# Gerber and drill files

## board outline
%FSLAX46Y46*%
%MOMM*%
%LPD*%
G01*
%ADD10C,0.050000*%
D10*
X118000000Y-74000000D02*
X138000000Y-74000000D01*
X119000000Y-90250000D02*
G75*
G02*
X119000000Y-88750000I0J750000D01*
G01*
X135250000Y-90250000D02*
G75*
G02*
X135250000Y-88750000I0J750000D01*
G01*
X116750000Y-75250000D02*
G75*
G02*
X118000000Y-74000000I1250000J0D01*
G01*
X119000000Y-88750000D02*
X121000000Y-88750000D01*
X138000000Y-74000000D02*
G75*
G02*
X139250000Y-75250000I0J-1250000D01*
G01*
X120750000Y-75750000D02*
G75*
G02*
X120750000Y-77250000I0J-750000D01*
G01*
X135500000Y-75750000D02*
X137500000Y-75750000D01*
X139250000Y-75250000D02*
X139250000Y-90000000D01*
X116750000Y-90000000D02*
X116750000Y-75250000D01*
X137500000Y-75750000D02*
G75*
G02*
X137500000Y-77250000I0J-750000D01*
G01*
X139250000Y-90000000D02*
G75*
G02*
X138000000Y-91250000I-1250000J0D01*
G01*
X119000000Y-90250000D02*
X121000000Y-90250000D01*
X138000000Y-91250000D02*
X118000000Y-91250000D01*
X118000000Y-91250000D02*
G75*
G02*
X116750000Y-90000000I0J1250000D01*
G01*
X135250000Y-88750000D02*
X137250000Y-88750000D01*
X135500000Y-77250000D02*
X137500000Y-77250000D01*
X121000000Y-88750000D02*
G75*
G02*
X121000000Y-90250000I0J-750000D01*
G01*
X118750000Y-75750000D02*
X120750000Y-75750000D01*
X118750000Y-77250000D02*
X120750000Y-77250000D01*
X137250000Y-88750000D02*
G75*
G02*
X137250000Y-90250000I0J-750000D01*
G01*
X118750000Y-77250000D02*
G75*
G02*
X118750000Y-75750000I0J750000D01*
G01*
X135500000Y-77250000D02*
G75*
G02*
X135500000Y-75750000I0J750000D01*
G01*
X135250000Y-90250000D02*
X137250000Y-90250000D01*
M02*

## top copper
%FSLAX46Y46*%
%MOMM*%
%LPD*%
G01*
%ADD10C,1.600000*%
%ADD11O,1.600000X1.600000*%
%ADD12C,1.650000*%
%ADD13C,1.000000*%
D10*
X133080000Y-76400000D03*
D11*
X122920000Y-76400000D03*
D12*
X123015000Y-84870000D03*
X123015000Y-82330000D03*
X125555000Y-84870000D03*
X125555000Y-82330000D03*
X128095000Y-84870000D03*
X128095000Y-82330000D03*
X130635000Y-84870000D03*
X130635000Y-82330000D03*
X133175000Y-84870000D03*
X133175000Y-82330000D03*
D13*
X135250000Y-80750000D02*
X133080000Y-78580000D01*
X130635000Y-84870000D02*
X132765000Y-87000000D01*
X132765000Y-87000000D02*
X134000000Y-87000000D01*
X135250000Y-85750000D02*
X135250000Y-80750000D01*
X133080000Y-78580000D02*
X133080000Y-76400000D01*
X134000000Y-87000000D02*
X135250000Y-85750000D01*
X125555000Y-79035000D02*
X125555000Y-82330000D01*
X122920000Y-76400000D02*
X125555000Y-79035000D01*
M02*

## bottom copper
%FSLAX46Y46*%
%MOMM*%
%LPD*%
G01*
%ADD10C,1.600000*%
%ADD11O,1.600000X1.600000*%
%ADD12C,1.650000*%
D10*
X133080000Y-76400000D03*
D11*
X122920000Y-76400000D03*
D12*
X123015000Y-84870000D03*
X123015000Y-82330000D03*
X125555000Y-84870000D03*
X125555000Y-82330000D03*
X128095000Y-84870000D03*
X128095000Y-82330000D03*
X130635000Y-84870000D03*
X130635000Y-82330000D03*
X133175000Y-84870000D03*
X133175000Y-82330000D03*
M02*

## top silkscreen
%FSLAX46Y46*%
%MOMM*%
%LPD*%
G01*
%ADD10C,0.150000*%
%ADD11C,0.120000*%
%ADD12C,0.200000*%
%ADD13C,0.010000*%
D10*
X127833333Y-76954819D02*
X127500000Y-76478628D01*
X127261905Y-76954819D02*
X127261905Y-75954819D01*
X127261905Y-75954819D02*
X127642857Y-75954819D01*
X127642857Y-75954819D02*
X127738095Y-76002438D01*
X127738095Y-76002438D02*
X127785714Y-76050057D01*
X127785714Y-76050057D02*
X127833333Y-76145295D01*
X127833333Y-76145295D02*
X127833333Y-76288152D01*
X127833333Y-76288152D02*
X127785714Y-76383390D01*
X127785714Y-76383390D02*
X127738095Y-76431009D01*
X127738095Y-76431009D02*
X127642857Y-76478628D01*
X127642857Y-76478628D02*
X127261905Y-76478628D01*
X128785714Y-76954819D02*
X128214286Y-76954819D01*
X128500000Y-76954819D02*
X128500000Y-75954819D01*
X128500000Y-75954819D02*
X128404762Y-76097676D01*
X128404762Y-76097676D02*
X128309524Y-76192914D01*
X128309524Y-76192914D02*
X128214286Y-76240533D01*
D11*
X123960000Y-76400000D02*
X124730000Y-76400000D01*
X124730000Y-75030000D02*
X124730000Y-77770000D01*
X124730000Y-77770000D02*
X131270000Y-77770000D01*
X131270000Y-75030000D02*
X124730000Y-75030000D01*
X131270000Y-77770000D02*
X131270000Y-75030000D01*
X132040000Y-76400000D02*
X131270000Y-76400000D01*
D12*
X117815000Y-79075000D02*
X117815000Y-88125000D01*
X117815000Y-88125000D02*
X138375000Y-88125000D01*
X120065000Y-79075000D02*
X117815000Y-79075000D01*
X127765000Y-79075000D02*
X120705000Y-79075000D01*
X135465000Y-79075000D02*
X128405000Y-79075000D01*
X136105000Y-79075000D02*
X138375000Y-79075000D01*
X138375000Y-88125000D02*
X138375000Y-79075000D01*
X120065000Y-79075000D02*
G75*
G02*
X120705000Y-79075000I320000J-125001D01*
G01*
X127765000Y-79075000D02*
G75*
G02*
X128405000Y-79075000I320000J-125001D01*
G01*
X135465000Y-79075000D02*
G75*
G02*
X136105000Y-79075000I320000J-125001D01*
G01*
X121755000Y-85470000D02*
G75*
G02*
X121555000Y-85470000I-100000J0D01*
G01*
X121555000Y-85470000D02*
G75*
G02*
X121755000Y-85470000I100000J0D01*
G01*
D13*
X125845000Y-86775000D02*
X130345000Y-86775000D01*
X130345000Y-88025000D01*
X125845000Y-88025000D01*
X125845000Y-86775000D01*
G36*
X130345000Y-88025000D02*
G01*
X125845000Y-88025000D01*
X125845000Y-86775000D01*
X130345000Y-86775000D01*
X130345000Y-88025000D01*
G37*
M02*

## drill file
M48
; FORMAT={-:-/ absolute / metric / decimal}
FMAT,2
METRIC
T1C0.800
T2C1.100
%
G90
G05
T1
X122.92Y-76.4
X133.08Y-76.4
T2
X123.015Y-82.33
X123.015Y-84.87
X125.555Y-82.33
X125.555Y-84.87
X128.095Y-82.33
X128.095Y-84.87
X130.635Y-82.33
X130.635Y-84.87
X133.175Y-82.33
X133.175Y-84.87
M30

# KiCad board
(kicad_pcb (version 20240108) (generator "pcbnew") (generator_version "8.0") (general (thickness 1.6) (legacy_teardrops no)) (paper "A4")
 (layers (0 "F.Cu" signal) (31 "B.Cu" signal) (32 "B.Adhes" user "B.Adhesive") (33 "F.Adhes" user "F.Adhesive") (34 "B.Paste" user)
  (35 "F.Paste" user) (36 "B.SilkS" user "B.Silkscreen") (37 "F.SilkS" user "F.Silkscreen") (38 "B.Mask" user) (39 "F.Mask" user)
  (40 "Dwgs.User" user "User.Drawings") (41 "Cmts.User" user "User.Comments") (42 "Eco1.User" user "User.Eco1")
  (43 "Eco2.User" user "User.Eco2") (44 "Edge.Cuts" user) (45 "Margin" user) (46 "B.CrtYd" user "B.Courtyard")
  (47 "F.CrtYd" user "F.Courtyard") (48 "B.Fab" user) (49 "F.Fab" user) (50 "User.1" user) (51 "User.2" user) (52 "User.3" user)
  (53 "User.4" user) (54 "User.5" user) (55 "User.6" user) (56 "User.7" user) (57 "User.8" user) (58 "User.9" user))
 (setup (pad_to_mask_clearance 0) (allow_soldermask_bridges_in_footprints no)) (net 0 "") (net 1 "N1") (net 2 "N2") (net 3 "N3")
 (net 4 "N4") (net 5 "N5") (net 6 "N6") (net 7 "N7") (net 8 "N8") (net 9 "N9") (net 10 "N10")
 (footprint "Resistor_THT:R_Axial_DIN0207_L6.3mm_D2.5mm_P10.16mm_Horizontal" (layer "F.Cu") (at 133.08 76.4 180)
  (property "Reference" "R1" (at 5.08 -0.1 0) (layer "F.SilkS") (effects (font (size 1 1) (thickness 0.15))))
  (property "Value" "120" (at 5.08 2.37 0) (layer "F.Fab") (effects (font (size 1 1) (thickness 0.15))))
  (fp_line (start 9.12 0) (end 8.35 0) (stroke (width 0.12) (type solid)) (layer "F.SilkS"))
  (fp_line (start 8.35 1.37) (end 8.35 -1.37) (stroke (width 0.12) (type solid)) (layer "F.SilkS"))
  (fp_line (start 8.35 -1.37) (end 1.81 -1.37) (stroke (width 0.12) (type solid)) (layer "F.SilkS"))
  (fp_line (start 1.81 1.37) (end 8.35 1.37) (stroke (width 0.12) (type solid)) (layer "F.SilkS"))
  (fp_line (start 1.81 -1.37) (end 1.81 1.37) (stroke (width 0.12) (type solid)) (layer "F.SilkS"))
  (fp_line (start 1.04 0) (end 1.81 0) (stroke (width 0.12) (type solid)) (layer "F.SilkS"))
  (pad "1" thru_hole circle (at 0 0 180) (size 1.6 1.6) (drill 0.8) (layers "*.Cu" "*.Mask") (remove_unused_layers no) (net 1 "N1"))
  (pad "2" thru_hole oval (at 10.16 0 180) (size 1.6 1.6) (drill 0.8) (layers "*.Cu" "*.Mask") (remove_unused_layers no) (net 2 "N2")))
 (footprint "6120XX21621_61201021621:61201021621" (layer "F.Cu") (at 128.095 83.6)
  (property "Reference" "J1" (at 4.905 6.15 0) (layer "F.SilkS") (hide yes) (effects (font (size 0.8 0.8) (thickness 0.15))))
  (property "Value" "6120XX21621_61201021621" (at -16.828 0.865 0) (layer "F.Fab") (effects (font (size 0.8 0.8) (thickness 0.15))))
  (fp_line (start -10.28 -4.525) (end -10.28 4.525) (stroke (width 0.2) (type solid)) (layer "F.SilkS"))
  (fp_line (start -10.28 4.525) (end 10.28 4.525) (stroke (width 0.2) (type solid)) (layer "F.SilkS"))
  (fp_line (start -8.03 -4.525) (end -10.28 -4.525) (stroke (width 0.2) (type solid)) (layer "F.SilkS"))
  (fp_line (start -0.33 -4.525) (end -7.39 -4.525) (stroke (width 0.2) (type solid)) (layer "F.SilkS"))
  (fp_line (start 7.37 -4.525) (end 0.31 -4.525) (stroke (width 0.2) (type solid)) (layer "F.SilkS"))
  (fp_line (start 8.01 -4.525) (end 10.28 -4.525) (stroke (width 0.2) (type solid)) (layer "F.SilkS"))
  (fp_line (start 10.28 4.525) (end 10.28 -4.525) (stroke (width 0.2) (type solid)) (layer "F.SilkS"))
  (fp_arc (start -8.03 -4.525) (mid -7.71 -4.743547) (end -7.39 -4.525) (stroke (width 0.2) (type solid)) (layer "F.SilkS"))
  (fp_arc (start -0.33 -4.525) (mid -0.01 -4.743547) (end 0.31 -4.525) (stroke (width 0.2) (type solid)) (layer "F.SilkS"))
  (fp_arc (start 7.37 -4.525) (mid 7.69 -4.743547) (end 8.01 -4.525) (stroke (width 0.2) (type solid)) (layer "F.SilkS"))
  (fp_circle (center -6.44 1.87) (end -6.34 1.87) (stroke (width 0.2) (type solid)) (fill none) (layer "F.SilkS"))
  (fp_poly
   (pts (xy -2.25 3.175) (xy 2.25 3.175) (xy 2.25 4.425) (xy -2.25 4.425)) (stroke (width 0.01) (type solid)) (fill solid) (layer "F.SilkS"))
  (pad "1" thru_hole circle (at -5.08 1.27) (size 1.65 1.65) (drill 1.1) (layers "*.Cu" "*.Mask") (remove_unused_layers no) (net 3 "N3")
   (solder_mask_margin 0.102))
  (pad "2" thru_hole circle (at -5.08 -1.27) (size 1.65 1.65) (drill 1.1) (layers "*.Cu" "*.Mask") (remove_unused_layers no) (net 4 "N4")
   (solder_mask_margin 0.102))
  (pad "3" thru_hole circle (at -2.54 1.27) (size 1.65 1.65) (drill 1.1) (layers "*.Cu" "*.Mask") (remove_unused_layers no) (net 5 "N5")
   (solder_mask_margin 0.102))
  (pad "4" thru_hole circle (at -2.54 -1.27) (size 1.65 1.65) (drill 1.1) (layers "*.Cu" "*.Mask") (remove_unused_layers no) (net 2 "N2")
   (solder_mask_margin 0.102))
  (pad "5" thru_hole circle (at 0 1.27) (size 1.65 1.65) (drill 1.1) (layers "*.Cu" "*.Mask") (remove_unused_layers no) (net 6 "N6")
   (solder_mask_margin 0.102))
  (pad "6" thru_hole circle (at 0 -1.27) (size 1.65 1.65) (drill 1.1) (layers "*.Cu" "*.Mask") (remove_unused_layers no) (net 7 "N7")
   (solder_mask_margin 0.102))
  (pad "7" thru_hole circle (at 2.54 1.27) (size 1.65 1.65) (drill 1.1) (layers "*.Cu" "*.Mask") (remove_unused_layers no) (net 1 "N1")
   (solder_mask_margin 0.102))
  (pad "8" thru_hole circle (at 2.54 -1.27) (size 1.65 1.65) (drill 1.1) (layers "*.Cu" "*.Mask") (remove_unused_layers no) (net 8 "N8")
   (solder_mask_margin 0.102))
  (pad "9" thru_hole circle (at 5.08 1.27) (size 1.65 1.65) (drill 1.1) (layers "*.Cu" "*.Mask") (remove_unused_layers no) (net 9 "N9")
   (solder_mask_margin 0.102))
  (pad "10" thru_hole circle (at 5.08 -1.27) (size 1.65 1.65) (drill 1.1) (layers "*.Cu" "*.Mask") (remove_unused_layers no) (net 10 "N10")
   (solder_mask_margin 0.102)))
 (gr_line (start 118 74) (end 138 74) (stroke (width 0.05) (type default)) (layer "Edge.Cuts"))
 (gr_arc (start 119 90.25) (mid 118.25 89.5) (end 119 88.75) (stroke (width 0.05) (type default)) (layer "Edge.Cuts"))
 (gr_arc (start 135.25 90.25) (mid 134.5 89.5) (end 135.25 88.75) (stroke (width 0.05) (type default)) (layer "Edge.Cuts"))
 (gr_arc (start 116.75 75.25) (mid 117.116117 74.366117) (end 118 74) (stroke (width 0.05) (type default)) (layer "Edge.Cuts"))
 (gr_line (start 119 88.75) (end 121 88.75) (stroke (width 0.05) (type default)) (layer "Edge.Cuts"))
 (gr_arc (start 138 74) (mid 138.883883 74.366117) (end 139.25 75.25) (stroke (width 0.05) (type default)) (layer "Edge.Cuts"))
 (gr_arc (start 120.75 75.75) (mid 121.5 76.5) (end 120.75 77.25) (stroke (width 0.05) (type default)) (layer "Edge.Cuts"))
 (gr_line (start 135.5 75.75) (end 137.5 75.75) (stroke (width 0.05) (type default)) (layer "Edge.Cuts"))
 (gr_line (start 139.25 75.25) (end 139.25 90) (stroke (width 0.05) (type default)) (layer "Edge.Cuts"))
 (gr_line (start 116.75 90) (end 116.75 75.25) (stroke (width 0.05) (type default)) (layer "Edge.Cuts"))
 (gr_arc (start 137.5 75.75) (mid 138.25 76.5) (end 137.5 77.25) (stroke (width 0.05) (type default)) (layer "Edge.Cuts"))
 (gr_arc (start 139.25 90) (mid 138.883883 90.883883) (end 138 91.25) (stroke (width 0.05) (type default)) (layer "Edge.Cuts"))
 (gr_line (start 119 90.25) (end 121 90.25) (stroke (width 0.05) (type default)) (layer "Edge.Cuts"))
 (gr_line (start 138 91.25) (end 118 91.25) (stroke (width 0.05) (type default)) (layer "Edge.Cuts"))
 (gr_arc (start 118 91.25) (mid 117.116117 90.883883) (end 116.75 90) (stroke (width 0.05) (type default)) (layer "Edge.Cuts"))
 (gr_line (start 135.25 88.75) (end 137.25 88.75) (stroke (width 0.05) (type default)) (layer "Edge.Cuts"))
 (gr_line (start 135.5 77.25) (end 137.5 77.25) (stroke (width 0.05) (type default)) (layer "Edge.Cuts"))
 (gr_arc (start 121 88.75) (mid 121.75 89.5) (end 121 90.25) (stroke (width 0.05) (type default)) (layer "Edge.Cuts"))
 (gr_line (start 118.75 75.75) (end 120.75 75.75) (stroke (width 0.05) (type default)) (layer "Edge.Cuts"))
 (gr_line (start 118.75 77.25) (end 120.75 77.25) (stroke (width 0.05) (type default)) (layer "Edge.Cuts"))
 (gr_arc (start 137.25 88.75) (mid 138 89.5) (end 137.25 90.25) (stroke (width 0.05) (type default)) (layer "Edge.Cuts"))
 (gr_arc (start 118.75 77.25) (mid 118 76.5) (end 118.75 75.75) (stroke (width 0.05) (type default)) (layer "Edge.Cuts"))
 (gr_arc (start 135.5 77.25) (mid 134.75 76.5) (end 135.5 75.75) (stroke (width 0.05) (type default)) (layer "Edge.Cuts"))
 (gr_line (start 135.25 90.25) (end 137.25 90.25) (stroke (width 0.05) (type default)) (layer "Edge.Cuts"))
 (segment (start 135.25 80.75) (end 133.08 78.58) (width 1) (layer "F.Cu") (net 1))
 (segment (start 130.635 84.87) (end 132.765 87) (width 1) (layer "F.Cu") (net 1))
 (segment (start 132.765 87) (end 134 87) (width 1) (layer "F.Cu") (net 1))
 (segment (start 135.25 85.75) (end 135.25 80.75) (width 1) (layer "F.Cu") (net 1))
 (segment (start 133.08 78.58) (end 133.08 76.4) (width 1) (layer "F.Cu") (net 1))
 (segment (start 134 87) (end 135.25 85.75) (width 1) (layer "F.Cu") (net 1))
 (segment (start 125.555 79.035) (end 125.555 82.33) (width 1) (layer "F.Cu") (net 2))
 (segment (start 122.92 76.4) (end 125.555 79.035) (width 1) (layer "F.Cu") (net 2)))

